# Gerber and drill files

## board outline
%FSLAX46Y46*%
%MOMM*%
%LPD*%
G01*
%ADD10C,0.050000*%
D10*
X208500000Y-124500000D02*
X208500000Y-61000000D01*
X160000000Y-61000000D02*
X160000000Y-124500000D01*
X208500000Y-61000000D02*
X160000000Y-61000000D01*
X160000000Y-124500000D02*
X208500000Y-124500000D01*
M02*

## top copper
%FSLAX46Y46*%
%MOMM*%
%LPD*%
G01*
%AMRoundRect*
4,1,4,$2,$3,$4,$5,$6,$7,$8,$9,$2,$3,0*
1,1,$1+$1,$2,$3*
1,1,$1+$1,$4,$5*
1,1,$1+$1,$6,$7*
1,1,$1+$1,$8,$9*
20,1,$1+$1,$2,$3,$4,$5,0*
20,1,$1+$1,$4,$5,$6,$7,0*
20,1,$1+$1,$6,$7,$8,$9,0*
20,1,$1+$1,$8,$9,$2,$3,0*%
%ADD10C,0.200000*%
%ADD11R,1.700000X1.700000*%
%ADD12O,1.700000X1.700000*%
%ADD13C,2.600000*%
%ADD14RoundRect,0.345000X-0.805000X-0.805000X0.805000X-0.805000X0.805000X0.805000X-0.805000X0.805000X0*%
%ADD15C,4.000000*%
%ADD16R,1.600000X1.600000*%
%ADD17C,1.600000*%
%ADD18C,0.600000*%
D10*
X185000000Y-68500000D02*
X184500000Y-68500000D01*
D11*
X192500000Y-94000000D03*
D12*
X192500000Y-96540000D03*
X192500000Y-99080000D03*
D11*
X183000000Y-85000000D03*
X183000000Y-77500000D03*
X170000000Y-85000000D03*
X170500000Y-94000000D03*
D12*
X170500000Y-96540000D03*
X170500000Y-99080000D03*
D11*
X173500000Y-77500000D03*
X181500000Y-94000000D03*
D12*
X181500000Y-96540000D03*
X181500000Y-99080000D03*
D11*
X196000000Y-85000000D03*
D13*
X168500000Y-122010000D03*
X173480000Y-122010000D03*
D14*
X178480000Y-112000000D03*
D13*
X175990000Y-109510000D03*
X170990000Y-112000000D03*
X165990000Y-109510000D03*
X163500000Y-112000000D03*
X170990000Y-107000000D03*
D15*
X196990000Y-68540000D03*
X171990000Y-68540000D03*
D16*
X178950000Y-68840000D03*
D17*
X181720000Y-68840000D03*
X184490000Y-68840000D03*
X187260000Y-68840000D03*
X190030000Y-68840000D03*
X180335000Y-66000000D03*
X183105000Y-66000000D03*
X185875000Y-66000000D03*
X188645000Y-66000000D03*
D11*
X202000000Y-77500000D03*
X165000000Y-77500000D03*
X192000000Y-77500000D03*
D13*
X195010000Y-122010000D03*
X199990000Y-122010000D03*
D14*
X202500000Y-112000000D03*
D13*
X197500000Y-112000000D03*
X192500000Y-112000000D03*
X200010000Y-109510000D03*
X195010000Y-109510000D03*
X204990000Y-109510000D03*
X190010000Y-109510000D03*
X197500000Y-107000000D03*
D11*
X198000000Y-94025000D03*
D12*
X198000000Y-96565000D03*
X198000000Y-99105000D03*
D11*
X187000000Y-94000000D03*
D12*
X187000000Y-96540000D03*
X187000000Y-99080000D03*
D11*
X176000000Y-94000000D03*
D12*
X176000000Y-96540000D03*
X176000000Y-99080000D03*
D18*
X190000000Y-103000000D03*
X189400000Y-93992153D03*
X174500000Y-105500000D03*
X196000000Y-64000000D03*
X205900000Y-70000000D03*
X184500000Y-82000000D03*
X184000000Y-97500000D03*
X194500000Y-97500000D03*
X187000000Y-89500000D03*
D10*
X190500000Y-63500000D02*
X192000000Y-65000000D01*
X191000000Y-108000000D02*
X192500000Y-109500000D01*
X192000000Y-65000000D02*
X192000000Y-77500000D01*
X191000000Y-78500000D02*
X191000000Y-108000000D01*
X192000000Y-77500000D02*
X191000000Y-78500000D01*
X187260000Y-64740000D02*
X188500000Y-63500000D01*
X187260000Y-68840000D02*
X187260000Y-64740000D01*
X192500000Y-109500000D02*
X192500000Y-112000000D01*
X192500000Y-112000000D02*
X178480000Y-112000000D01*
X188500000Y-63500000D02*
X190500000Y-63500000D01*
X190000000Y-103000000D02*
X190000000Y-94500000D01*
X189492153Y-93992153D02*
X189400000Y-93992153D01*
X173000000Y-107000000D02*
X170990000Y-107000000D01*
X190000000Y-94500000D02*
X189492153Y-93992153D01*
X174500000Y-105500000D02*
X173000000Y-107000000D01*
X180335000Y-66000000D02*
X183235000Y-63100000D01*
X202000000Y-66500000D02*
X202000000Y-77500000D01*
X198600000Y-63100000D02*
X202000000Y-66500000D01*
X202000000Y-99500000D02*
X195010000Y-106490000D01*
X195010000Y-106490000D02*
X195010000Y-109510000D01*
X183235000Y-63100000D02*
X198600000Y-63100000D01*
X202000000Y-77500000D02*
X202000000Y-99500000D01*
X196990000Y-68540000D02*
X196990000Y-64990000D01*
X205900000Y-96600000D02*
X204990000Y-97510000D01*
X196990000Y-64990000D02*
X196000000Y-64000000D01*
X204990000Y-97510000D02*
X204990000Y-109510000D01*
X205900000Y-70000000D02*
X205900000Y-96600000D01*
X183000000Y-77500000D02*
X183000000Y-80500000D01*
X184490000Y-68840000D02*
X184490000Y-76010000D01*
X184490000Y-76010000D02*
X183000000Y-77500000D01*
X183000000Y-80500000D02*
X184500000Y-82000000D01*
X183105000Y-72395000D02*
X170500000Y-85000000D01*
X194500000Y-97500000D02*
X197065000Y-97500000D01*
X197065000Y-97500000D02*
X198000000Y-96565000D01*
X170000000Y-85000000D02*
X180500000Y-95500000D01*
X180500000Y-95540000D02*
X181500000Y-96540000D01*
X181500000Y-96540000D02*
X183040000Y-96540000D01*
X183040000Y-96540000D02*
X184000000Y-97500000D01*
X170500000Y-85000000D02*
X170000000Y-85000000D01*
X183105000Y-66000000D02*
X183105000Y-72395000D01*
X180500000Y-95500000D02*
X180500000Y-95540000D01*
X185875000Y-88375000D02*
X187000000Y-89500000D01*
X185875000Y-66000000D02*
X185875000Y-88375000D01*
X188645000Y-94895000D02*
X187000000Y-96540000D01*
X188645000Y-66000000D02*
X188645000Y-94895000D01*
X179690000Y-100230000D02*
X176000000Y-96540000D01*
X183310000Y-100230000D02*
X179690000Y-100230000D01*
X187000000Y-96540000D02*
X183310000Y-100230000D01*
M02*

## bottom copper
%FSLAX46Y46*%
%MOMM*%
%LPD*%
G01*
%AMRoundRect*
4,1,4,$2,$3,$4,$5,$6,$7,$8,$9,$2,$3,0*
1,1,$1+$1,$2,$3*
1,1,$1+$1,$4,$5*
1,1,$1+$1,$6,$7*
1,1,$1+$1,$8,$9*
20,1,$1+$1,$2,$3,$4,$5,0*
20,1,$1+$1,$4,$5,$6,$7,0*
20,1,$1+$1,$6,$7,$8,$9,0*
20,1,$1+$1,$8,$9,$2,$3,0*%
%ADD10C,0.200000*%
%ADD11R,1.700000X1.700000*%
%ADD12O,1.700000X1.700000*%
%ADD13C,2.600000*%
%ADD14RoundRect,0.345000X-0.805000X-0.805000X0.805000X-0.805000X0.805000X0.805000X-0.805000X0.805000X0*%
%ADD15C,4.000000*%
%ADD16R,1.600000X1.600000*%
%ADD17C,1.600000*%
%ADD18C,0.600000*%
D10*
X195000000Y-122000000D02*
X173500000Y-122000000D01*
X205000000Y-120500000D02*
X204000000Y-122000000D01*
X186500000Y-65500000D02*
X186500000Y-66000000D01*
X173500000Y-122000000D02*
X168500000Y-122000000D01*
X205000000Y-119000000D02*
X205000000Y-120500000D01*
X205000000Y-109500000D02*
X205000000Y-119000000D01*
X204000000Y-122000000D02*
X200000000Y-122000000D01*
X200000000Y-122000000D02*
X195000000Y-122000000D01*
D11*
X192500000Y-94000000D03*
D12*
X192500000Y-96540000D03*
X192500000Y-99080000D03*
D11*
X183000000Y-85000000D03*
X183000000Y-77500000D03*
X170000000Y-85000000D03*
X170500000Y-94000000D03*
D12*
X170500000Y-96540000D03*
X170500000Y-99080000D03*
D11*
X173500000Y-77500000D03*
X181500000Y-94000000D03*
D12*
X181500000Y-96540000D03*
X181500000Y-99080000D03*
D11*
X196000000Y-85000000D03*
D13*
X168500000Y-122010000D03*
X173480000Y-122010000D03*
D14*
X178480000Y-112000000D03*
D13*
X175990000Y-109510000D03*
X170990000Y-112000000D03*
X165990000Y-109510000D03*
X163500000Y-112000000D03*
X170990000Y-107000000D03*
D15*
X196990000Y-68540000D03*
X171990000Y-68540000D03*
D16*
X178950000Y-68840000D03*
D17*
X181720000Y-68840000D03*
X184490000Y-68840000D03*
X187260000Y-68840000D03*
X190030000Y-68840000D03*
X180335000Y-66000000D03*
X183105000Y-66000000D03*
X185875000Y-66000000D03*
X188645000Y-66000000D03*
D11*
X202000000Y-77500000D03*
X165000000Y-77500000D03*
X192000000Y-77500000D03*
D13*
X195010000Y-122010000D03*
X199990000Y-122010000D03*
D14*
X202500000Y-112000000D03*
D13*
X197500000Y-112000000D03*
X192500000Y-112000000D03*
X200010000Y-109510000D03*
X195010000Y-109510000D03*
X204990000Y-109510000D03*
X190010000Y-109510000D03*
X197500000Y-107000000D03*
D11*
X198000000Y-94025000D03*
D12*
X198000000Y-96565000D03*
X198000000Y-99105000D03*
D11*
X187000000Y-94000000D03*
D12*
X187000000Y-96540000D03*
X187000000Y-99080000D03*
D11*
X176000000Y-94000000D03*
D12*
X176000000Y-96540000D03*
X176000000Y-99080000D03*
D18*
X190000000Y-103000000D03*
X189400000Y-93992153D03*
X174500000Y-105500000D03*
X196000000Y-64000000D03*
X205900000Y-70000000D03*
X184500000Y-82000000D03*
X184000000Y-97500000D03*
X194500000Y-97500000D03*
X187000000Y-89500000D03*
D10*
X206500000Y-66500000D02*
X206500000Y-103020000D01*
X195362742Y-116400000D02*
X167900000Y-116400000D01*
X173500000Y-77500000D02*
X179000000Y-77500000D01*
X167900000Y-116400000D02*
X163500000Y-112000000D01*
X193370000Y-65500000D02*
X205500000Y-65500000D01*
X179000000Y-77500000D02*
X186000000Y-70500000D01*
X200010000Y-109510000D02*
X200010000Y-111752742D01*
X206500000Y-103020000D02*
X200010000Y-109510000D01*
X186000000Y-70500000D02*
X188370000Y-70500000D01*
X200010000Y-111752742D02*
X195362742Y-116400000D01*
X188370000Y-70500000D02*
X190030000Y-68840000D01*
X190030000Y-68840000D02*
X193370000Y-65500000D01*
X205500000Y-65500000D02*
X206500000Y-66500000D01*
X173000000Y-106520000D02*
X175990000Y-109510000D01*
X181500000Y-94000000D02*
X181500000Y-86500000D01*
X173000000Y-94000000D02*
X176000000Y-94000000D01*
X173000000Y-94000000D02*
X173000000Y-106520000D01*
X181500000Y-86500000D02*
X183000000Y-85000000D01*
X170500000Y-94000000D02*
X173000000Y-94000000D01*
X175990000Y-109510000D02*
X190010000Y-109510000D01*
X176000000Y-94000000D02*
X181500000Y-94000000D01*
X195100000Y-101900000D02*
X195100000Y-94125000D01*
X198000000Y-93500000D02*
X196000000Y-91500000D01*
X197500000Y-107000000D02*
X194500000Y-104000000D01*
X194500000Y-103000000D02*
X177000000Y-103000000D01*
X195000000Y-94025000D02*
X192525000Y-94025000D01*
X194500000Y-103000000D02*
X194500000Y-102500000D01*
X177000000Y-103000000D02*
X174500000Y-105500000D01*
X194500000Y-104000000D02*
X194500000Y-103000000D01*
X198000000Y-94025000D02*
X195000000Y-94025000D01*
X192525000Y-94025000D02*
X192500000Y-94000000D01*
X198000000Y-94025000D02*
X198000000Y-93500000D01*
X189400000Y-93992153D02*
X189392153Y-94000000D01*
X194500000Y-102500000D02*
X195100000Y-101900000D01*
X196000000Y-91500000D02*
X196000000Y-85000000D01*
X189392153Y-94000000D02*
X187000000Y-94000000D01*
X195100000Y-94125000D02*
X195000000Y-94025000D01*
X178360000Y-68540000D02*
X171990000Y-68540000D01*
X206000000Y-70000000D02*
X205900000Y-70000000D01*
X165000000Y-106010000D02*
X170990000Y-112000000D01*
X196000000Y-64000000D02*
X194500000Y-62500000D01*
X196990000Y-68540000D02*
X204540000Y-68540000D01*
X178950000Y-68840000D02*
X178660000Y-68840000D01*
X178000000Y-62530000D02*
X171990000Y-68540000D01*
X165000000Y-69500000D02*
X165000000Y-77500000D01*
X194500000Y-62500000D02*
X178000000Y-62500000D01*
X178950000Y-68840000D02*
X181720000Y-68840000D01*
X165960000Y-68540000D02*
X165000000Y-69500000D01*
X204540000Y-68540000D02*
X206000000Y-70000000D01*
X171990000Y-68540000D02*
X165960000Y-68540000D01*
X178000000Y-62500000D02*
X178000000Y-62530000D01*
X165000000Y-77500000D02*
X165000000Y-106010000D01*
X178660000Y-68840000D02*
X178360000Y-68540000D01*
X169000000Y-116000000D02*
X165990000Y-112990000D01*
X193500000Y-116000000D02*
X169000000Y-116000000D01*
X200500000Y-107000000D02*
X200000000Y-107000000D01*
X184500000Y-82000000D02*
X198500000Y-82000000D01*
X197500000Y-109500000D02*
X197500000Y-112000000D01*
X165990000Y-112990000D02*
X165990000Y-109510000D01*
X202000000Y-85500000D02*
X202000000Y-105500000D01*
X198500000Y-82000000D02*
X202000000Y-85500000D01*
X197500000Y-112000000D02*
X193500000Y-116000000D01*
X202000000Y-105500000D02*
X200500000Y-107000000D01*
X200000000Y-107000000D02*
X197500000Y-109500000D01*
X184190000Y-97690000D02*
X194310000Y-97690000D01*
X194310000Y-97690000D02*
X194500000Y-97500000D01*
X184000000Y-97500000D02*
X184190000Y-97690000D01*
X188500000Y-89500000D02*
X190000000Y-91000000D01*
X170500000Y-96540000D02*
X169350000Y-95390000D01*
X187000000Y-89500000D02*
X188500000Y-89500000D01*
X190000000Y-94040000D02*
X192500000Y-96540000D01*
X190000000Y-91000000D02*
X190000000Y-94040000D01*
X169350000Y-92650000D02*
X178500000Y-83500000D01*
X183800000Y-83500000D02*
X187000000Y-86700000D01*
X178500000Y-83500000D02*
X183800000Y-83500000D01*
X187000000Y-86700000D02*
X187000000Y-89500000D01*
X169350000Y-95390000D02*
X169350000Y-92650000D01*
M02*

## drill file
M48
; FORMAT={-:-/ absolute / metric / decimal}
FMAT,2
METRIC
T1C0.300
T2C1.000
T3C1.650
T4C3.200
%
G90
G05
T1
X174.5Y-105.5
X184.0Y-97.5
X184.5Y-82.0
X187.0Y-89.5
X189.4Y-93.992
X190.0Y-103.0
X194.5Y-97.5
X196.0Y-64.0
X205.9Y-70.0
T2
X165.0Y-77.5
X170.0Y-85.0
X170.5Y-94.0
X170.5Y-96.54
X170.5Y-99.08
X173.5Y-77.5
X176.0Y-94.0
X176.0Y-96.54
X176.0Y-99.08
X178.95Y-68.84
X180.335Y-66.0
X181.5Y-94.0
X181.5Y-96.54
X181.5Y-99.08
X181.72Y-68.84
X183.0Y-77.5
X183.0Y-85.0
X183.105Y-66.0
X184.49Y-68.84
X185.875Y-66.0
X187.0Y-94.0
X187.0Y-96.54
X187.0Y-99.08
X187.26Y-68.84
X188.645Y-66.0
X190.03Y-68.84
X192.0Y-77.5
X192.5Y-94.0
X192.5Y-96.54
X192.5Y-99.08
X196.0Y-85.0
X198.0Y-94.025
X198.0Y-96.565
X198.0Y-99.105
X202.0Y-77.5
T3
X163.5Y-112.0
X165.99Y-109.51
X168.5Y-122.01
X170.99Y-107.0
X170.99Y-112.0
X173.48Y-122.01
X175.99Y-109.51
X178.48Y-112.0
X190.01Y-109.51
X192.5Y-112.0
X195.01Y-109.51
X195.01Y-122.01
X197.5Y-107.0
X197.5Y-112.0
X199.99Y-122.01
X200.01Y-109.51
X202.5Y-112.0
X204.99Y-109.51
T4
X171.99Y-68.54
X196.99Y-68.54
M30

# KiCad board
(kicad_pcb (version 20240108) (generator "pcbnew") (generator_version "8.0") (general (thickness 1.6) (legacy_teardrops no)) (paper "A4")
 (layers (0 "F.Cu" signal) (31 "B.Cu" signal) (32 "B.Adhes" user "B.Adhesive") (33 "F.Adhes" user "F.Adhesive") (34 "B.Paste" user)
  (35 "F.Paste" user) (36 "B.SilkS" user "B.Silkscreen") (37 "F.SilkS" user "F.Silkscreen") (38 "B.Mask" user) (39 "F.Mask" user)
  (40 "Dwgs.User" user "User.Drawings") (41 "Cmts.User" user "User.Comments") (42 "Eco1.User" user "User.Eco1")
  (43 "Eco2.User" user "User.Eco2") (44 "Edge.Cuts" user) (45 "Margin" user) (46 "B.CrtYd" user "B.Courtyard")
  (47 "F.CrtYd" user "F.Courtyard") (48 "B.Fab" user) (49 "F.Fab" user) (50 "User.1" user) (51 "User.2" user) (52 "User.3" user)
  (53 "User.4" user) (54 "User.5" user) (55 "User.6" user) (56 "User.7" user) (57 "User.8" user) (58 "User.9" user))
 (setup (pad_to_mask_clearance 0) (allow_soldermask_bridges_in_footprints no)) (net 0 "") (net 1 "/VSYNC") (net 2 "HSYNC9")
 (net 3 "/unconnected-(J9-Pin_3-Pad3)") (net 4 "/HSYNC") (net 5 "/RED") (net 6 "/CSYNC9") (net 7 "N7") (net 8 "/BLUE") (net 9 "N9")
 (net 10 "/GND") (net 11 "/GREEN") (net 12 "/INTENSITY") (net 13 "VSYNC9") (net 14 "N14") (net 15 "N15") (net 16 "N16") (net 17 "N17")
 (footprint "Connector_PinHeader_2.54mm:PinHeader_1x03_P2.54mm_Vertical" (layer "F.Cu") (at 192.5 94)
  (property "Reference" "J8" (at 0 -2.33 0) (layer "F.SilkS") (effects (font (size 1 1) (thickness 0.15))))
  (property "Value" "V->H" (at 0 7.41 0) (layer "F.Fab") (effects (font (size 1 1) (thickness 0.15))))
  (pad "1" thru_hole rect (at 0 0) (size 1.7 1.7) (drill 1) (layers "*.Cu" "*.Mask") (remove_unused_layers no) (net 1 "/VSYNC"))
  (pad "2" thru_hole oval (at 0 2.54) (size 1.7 1.7) (drill 1) (layers "*.Cu" "*.Mask") (remove_unused_layers no) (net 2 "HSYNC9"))
  (pad "3" thru_hole oval (at 0 5.08) (size 1.7 1.7) (drill 1) (layers "*.Cu" "*.Mask") (remove_unused_layers no)
   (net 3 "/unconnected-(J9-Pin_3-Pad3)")))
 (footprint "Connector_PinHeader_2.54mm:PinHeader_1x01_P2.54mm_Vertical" (layer "F.Cu") (at 183 85)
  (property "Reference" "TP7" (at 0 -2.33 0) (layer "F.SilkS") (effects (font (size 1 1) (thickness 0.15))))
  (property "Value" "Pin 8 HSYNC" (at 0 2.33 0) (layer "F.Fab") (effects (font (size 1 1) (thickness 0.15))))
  (pad "1" thru_hole rect (at 0 0) (size 1.7 1.7) (drill 1) (layers "*.Cu" "*.Mask") (remove_unused_layers no) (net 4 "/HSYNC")))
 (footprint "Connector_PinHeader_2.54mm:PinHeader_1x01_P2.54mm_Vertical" (layer "F.Cu") (at 183 77.5)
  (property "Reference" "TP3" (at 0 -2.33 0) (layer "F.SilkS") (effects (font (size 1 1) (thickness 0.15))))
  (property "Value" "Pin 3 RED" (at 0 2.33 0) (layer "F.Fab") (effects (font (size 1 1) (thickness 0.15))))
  (pad "1" thru_hole rect (at 0 0) (size 1.7 1.7) (drill 1) (layers "*.Cu" "*.Mask") (remove_unused_layers no) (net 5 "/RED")))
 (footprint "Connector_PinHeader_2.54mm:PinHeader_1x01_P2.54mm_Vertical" (layer "F.Cu") (at 170 85)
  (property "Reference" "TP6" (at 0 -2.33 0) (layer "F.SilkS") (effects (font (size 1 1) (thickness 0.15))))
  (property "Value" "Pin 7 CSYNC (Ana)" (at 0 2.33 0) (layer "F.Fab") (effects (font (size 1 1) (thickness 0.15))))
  (pad "1" thru_hole rect (at 0 0) (size 1.7 1.7) (drill 1) (layers "*.Cu" "*.Mask") (remove_unused_layers no) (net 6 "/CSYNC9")))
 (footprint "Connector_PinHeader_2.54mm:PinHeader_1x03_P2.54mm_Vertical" (layer "F.Cu") (at 170.5 94)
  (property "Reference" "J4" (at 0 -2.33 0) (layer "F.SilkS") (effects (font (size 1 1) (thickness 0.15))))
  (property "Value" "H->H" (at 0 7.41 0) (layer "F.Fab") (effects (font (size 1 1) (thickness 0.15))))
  (pad "1" thru_hole rect (at 0 0) (size 1.7 1.7) (drill 1) (layers "*.Cu" "*.Mask") (remove_unused_layers no) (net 4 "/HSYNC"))
  (pad "2" thru_hole oval (at 0 2.54) (size 1.7 1.7) (drill 1) (layers "*.Cu" "*.Mask") (remove_unused_layers no) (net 2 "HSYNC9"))
  (pad "3" thru_hole oval (at 0 5.08) (size 1.7 1.7) (drill 1) (layers "*.Cu" "*.Mask") (remove_unused_layers no) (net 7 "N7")))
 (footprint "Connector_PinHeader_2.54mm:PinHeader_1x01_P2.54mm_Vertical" (layer "F.Cu") (at 173.5 77.5)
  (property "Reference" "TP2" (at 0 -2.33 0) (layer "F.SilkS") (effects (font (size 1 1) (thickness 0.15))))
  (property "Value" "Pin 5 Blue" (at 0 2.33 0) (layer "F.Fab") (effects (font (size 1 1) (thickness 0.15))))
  (pad "1" thru_hole rect (at 0 0) (size 1.7 1.7) (drill 1) (layers "*.Cu" "*.Mask") (remove_unused_layers no) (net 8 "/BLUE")))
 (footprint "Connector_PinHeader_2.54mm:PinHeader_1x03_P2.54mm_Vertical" (layer "F.Cu") (at 181.5 94)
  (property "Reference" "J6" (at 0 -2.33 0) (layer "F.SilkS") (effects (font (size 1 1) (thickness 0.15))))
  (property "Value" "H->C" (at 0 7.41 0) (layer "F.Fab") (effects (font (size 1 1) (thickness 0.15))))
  (pad "1" thru_hole rect (at 0 0) (size 1.7 1.7) (drill 1) (layers "*.Cu" "*.Mask") (remove_unused_layers no) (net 4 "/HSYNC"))
  (pad "2" thru_hole oval (at 0 2.54) (size 1.7 1.7) (drill 1) (layers "*.Cu" "*.Mask") (remove_unused_layers no) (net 6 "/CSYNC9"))
  (pad "3" thru_hole oval (at 0 5.08) (size 1.7 1.7) (drill 1) (layers "*.Cu" "*.Mask") (remove_unused_layers no) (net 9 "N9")))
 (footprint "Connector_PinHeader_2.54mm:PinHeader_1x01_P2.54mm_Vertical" (layer "F.Cu") (at 196 85)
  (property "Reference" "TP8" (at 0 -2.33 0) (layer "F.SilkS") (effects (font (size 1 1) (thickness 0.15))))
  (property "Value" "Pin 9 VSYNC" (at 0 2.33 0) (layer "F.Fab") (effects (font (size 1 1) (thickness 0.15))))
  (pad "1" thru_hole rect (at 0 0) (size 1.7 1.7) (drill 1) (layers "*.Cu" "*.Mask") (remove_unused_layers no) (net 1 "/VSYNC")))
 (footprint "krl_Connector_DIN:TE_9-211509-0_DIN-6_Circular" (layer "F.Cu") (at 178.48 112)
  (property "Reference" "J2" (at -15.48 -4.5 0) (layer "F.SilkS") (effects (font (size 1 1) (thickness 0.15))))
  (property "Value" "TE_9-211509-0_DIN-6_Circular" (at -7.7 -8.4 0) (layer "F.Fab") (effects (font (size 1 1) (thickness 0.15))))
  (pad "0" thru_hole circle (at -9.98 10.01) (size 2.6 2.6) (drill 1.65) (layers "*.Cu" "*.Mask") (remove_unused_layers no) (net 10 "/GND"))
  (pad "0" thru_hole circle (at -5 10.01) (size 2.6 2.6) (drill 1.65) (layers "*.Cu" "*.Mask") (remove_unused_layers no) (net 10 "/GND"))
  (pad "1" thru_hole roundrect (at 0 0) (size 2.3 2.3) (drill 1.65) (layers "*.Cu" "*.Mask") (remove_unused_layers no)
   (roundrect_rratio 0.15) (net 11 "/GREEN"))
  (pad "2" thru_hole circle (at -2.49 -2.49) (size 2.6 2.6) (drill 1.65) (layers "*.Cu" "*.Mask") (remove_unused_layers no) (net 4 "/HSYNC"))
  (pad "3" thru_hole circle (at -7.49 0) (size 2.6 2.6) (drill 1.65) (layers "*.Cu" "*.Mask") (remove_unused_layers no) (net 10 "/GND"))
  (pad "4" thru_hole circle (at -12.49 -2.49) (size 2.6 2.6) (drill 1.65) (layers "*.Cu" "*.Mask") (remove_unused_layers no) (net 5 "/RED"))
  (pad "5" thru_hole circle (at -14.98 0) (size 2.6 2.6) (drill 1.65) (layers "*.Cu" "*.Mask") (remove_unused_layers no) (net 8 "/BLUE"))
  (pad "6" thru_hole circle (at -7.49 -5) (size 2.6 2.6) (drill 1.65) (layers "*.Cu" "*.Mask") (remove_unused_layers no) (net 1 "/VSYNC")))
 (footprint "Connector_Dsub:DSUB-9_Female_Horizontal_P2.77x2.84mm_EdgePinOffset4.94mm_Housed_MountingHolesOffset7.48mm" (layer "F.Cu")
  (at 178.95 68.84 180)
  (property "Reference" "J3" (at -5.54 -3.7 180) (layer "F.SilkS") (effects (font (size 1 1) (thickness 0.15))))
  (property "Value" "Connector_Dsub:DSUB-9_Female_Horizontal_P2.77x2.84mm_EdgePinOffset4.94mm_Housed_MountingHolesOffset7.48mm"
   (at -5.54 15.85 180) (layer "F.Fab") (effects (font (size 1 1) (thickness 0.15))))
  (pad "0" thru_hole circle (at -18.04 0.3 180) (size 4 4) (drill 3.2) (layers "*.Cu" "*.Mask") (remove_unused_layers no) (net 10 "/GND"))
  (pad "0" thru_hole circle (at 6.96 0.3 180) (size 4 4) (drill 3.2) (layers "*.Cu" "*.Mask") (remove_unused_layers no) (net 10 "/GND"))
  (pad "1" thru_hole rect (at 0 0 180) (size 1.6 1.6) (drill 1) (layers "*.Cu" "*.Mask") (remove_unused_layers no) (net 10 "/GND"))
  (pad "2" thru_hole circle (at -2.77 0 180) (size 1.6 1.6) (drill 1) (layers "*.Cu" "*.Mask") (remove_unused_layers no) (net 10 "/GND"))
  (pad "3" thru_hole circle (at -5.54 0 180) (size 1.6 1.6) (drill 1) (layers "*.Cu" "*.Mask") (remove_unused_layers no) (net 5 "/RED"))
  (pad "4" thru_hole circle (at -8.31 0 180) (size 1.6 1.6) (drill 1) (layers "*.Cu" "*.Mask") (remove_unused_layers no) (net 11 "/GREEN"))
  (pad "5" thru_hole circle (at -11.08 0 180) (size 1.6 1.6) (drill 1) (layers "*.Cu" "*.Mask") (remove_unused_layers no) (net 8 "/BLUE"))
  (pad "6" thru_hole circle (at -1.385 2.84 180) (size 1.6 1.6) (drill 1) (layers "*.Cu" "*.Mask") (remove_unused_layers no)
   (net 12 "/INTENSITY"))
  (pad "7" thru_hole circle (at -4.155 2.84 180) (size 1.6 1.6) (drill 1) (layers "*.Cu" "*.Mask") (remove_unused_layers no)
   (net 6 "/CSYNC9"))
  (pad "8" thru_hole circle (at -6.925 2.84 180) (size 1.6 1.6) (drill 1) (layers "*.Cu" "*.Mask") (remove_unused_layers no)
   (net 2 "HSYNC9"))
  (pad "9" thru_hole circle (at -9.695 2.84 180) (size 1.6 1.6) (drill 1) (layers "*.Cu" "*.Mask") (remove_unused_layers no)
   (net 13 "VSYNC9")))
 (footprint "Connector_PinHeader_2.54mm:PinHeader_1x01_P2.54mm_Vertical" (layer "F.Cu") (at 202 77.5)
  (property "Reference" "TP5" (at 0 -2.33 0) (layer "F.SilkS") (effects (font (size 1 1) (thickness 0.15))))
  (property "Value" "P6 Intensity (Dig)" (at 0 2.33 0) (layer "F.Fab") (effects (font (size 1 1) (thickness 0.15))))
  (pad "1" thru_hole rect (at 0 0) (size 1.7 1.7) (drill 1) (layers "*.Cu" "*.Mask") (remove_unused_layers no) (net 12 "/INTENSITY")))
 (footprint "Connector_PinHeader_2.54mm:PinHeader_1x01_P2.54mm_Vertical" (layer "F.Cu") (at 165 77.5)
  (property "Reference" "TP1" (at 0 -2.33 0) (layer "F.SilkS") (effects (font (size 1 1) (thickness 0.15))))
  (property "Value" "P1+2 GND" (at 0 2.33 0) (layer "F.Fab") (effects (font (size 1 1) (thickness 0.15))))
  (pad "1" thru_hole rect (at 0 0) (size 1.7 1.7) (drill 1) (layers "*.Cu" "*.Mask") (remove_unused_layers no) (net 10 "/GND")))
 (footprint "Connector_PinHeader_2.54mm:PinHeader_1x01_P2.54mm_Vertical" (layer "F.Cu") (at 192 77.5)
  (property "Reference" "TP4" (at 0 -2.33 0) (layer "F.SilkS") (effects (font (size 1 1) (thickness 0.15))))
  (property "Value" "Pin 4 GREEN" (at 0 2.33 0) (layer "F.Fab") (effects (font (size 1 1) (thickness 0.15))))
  (pad "1" thru_hole rect (at 0 0) (size 1.7 1.7) (drill 1) (layers "*.Cu" "*.Mask") (remove_unused_layers no) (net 11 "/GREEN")))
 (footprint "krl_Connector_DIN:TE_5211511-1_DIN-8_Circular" (layer "F.Cu") (at 202.5 112)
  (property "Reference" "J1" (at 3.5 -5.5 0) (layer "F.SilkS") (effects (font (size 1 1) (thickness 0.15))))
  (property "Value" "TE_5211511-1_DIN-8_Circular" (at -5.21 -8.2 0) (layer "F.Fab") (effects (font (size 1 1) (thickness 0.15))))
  (pad "0" thru_hole circle (at -7.49 10.01) (size 2.6 2.6) (drill 1.65) (layers "*.Cu" "*.Mask") (remove_unused_layers no) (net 10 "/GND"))
  (pad "0" thru_hole circle (at -2.51 10.01) (size 2.6 2.6) (drill 1.65) (layers "*.Cu" "*.Mask") (remove_unused_layers no) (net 10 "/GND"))
  (pad "1" thru_hole roundrect (at 0 0) (size 2.3 2.3) (drill 1.65) (layers "*.Cu" "*.Mask") (remove_unused_layers no)
   (roundrect_rratio 0.15) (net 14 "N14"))
  (pad "2" thru_hole circle (at -5 0) (size 2.6 2.6) (drill 1.65) (layers "*.Cu" "*.Mask") (remove_unused_layers no) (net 5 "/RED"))
  (pad "3" thru_hole circle (at -10 0) (size 2.6 2.6) (drill 1.65) (layers "*.Cu" "*.Mask") (remove_unused_layers no) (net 11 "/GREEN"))
  (pad "4" thru_hole circle (at -2.49 -2.49) (size 2.6 2.6) (drill 1.65) (layers "*.Cu" "*.Mask") (remove_unused_layers no) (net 8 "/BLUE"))
  (pad "5" thru_hole circle (at -7.49 -2.49) (size 2.6 2.6) (drill 1.65) (layers "*.Cu" "*.Mask") (remove_unused_layers no)
   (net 12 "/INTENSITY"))
  (pad "6" thru_hole circle (at 2.49 -2.49) (size 2.6 2.6) (drill 1.65) (layers "*.Cu" "*.Mask") (remove_unused_layers no) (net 10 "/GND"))
  (pad "7" thru_hole circle (at -12.49 -2.49) (size 2.6 2.6) (drill 1.65) (layers "*.Cu" "*.Mask") (remove_unused_layers no)
   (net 4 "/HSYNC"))
  (pad "8" thru_hole circle (at -5 -5) (size 2.6 2.6) (drill 1.65) (layers "*.Cu" "*.Mask") (remove_unused_layers no) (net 1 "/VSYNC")))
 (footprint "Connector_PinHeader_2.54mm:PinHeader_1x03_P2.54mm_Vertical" (layer "F.Cu") (at 198 94.025)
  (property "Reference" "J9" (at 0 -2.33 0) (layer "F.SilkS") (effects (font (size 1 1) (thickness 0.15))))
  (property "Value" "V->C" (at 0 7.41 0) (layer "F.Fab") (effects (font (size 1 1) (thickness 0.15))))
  (pad "1" thru_hole rect (at 0 0) (size 1.7 1.7) (drill 1) (layers "*.Cu" "*.Mask") (remove_unused_layers no) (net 1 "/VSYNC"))
  (pad "2" thru_hole oval (at 0 2.54) (size 1.7 1.7) (drill 1) (layers "*.Cu" "*.Mask") (remove_unused_layers no) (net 6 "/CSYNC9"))
  (pad "3" thru_hole oval (at 0 5.08) (size 1.7 1.7) (drill 1) (layers "*.Cu" "*.Mask") (remove_unused_layers no) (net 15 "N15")))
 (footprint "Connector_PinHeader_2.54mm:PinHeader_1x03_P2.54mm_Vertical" (layer "F.Cu") (at 187 94)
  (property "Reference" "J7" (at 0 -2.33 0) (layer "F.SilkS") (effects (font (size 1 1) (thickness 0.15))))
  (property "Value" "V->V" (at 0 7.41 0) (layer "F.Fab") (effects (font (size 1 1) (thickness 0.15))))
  (pad "1" thru_hole rect (at 0 0) (size 1.7 1.7) (drill 1) (layers "*.Cu" "*.Mask") (remove_unused_layers no) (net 1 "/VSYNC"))
  (pad "2" thru_hole oval (at 0 2.54) (size 1.7 1.7) (drill 1) (layers "*.Cu" "*.Mask") (remove_unused_layers no) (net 13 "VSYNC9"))
  (pad "3" thru_hole oval (at 0 5.08) (size 1.7 1.7) (drill 1) (layers "*.Cu" "*.Mask") (remove_unused_layers no) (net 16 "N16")))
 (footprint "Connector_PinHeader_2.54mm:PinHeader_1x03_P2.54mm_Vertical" (layer "F.Cu") (at 176 94)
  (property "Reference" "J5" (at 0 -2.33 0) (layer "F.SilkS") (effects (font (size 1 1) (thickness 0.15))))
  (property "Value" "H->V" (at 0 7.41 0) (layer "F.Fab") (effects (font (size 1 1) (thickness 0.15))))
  (pad "1" thru_hole rect (at 0 0) (size 1.7 1.7) (drill 1) (layers "*.Cu" "*.Mask") (remove_unused_layers no) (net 4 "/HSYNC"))
  (pad "2" thru_hole oval (at 0 2.54) (size 1.7 1.7) (drill 1) (layers "*.Cu" "*.Mask") (remove_unused_layers no) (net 13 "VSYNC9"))
  (pad "3" thru_hole oval (at 0 5.08) (size 1.7 1.7) (drill 1) (layers "*.Cu" "*.Mask") (remove_unused_layers no) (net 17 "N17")))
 (gr_line (start 185 68.5) (end 184.5 68.5) (stroke (width 0.2) (type default)) (layer "F.Cu") (net 5))
 (gr_line (start 195 122) (end 173.5 122) (stroke (width 0.2) (type default)) (layer "B.Cu") (net 10))
 (gr_line (start 205 120.5) (end 204 122) (stroke (width 0.2) (type default)) (layer "B.Cu") (net 10))
 (gr_line (start 186.5 65.5) (end 186.5 66) (stroke (width 0.2) (type default)) (layer "B.Cu") (net 2))
 (gr_line (start 173.5 122) (end 168.5 122) (stroke (width 0.2) (type default)) (layer "B.Cu") (net 10))
 (gr_line (start 205 119) (end 205 120.5) (stroke (width 0.2) (type default)) (layer "B.Cu") (net 10))
 (gr_line (start 205 109.5) (end 205 119) (stroke (width 0.2) (type default)) (layer "B.Cu") (net 10))
 (gr_line (start 204 122) (end 200 122) (stroke (width 0.2) (type default)) (layer "B.Cu") (net 10))
 (gr_line (start 200 122) (end 195 122) (stroke (width 0.2) (type default)) (layer "B.Cu") (net 10))
 (gr_line (start 208.5 124.5) (end 208.5 61) (stroke (width 0.05) (type default)) (layer "Edge.Cuts"))
 (gr_line (start 160 61) (end 160 124.5) (stroke (width 0.05) (type default)) (layer "Edge.Cuts"))
 (gr_line (start 208.5 61) (end 160 61) (stroke (width 0.05) (type default)) (layer "Edge.Cuts"))
 (gr_line (start 160 124.5) (end 208.5 124.5) (stroke (width 0.05) (type default)) (layer "Edge.Cuts"))
 (segment (start 206.5 66.5) (end 206.5 103.02) (width 0.2) (layer "B.Cu") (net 8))
 (segment (start 195.362742 116.4) (end 167.9 116.4) (width 0.2) (layer "B.Cu") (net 8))
 (segment (start 173.5 77.5) (end 179 77.5) (width 0.2) (layer "B.Cu") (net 8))
 (segment (start 167.9 116.4) (end 163.5 112) (width 0.2) (layer "B.Cu") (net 8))
 (segment (start 193.37 65.5) (end 205.5 65.5) (width 0.2) (layer "B.Cu") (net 8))
 (segment (start 179 77.5) (end 186 70.5) (width 0.2) (layer "B.Cu") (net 8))
 (segment (start 200.01 109.51) (end 200.01 111.752742) (width 0.2) (layer "B.Cu") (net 8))
 (segment (start 206.5 103.02) (end 200.01 109.51) (width 0.2) (layer "B.Cu") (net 8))
 (segment (start 186 70.5) (end 188.37 70.5) (width 0.2) (layer "B.Cu") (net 8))
 (segment (start 200.01 111.752742) (end 195.362742 116.4) (width 0.2) (layer "B.Cu") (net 8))
 (segment (start 188.37 70.5) (end 190.03 68.84) (width 0.2) (layer "B.Cu") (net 8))
 (segment (start 190.03 68.84) (end 193.37 65.5) (width 0.2) (layer "B.Cu") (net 8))
 (segment (start 205.5 65.5) (end 206.5 66.5) (width 0.2) (layer "B.Cu") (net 8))
 (segment (start 173 106.52) (end 175.99 109.51) (width 0.2) (layer "B.Cu") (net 4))
 (segment (start 181.5 94) (end 181.5 86.5) (width 0.2) (layer "B.Cu") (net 4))
 (segment (start 173 94) (end 176 94) (width 0.2) (layer "B.Cu") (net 4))
 (segment (start 173 94) (end 173 106.52) (width 0.2) (layer "B.Cu") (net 4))
 (segment (start 181.5 86.5) (end 183 85) (width 0.2) (layer "B.Cu") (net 4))
 (segment (start 170.5 94) (end 173 94) (width 0.2) (layer "B.Cu") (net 4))
 (segment (start 175.99 109.51) (end 190.01 109.51) (width 0.2) (layer "B.Cu") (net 4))
 (segment (start 176 94) (end 181.5 94) (width 0.2) (layer "B.Cu") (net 4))
 (segment (start 190.5 63.5) (end 192 65) (width 0.2) (layer "F.Cu") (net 11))
 (segment (start 191 108) (end 192.5 109.5) (width 0.2) (layer "F.Cu") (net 11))
 (segment (start 192 65) (end 192 77.5) (width 0.2) (layer "F.Cu") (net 11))
 (segment (start 191 78.5) (end 191 108) (width 0.2) (layer "F.Cu") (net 11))
 (segment (start 192 77.5) (end 191 78.5) (width 0.2) (layer "F.Cu") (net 11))
 (segment (start 187.26 64.74) (end 188.5 63.5) (width 0.2) (layer "F.Cu") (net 11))
 (segment (start 187.26 68.84) (end 187.26 64.74) (width 0.2) (layer "F.Cu") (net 11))
 (segment (start 192.5 109.5) (end 192.5 112) (width 0.2) (layer "F.Cu") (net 11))
 (segment (start 192.5 112) (end 178.48 112) (width 0.2) (layer "F.Cu") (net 11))
 (segment (start 188.5 63.5) (end 190.5 63.5) (width 0.2) (layer "F.Cu") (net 11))
 (segment (start 190 103) (end 190 94.5) (width 0.2) (layer "F.Cu") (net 1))
 (segment (start 189.492153 93.992153) (end 189.4 93.992153) (width 0.2) (layer "F.Cu") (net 1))
 (segment (start 173 107) (end 170.99 107) (width 0.2) (layer "F.Cu") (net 1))
 (segment (start 190 94.5) (end 189.492153 93.992153) (width 0.2) (layer "F.Cu") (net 1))
 (segment (start 174.5 105.5) (end 173 107) (width 0.2) (layer "F.Cu") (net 1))
 (via (at 190 103) (size 0.6) (drill 0.3) (layers "F.Cu" "B.Cu") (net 1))
 (via (at 189.4 93.992153) (size 0.6) (drill 0.3) (layers "F.Cu" "B.Cu") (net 1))
 (via (at 174.5 105.5) (size 0.6) (drill 0.3) (layers "F.Cu" "B.Cu") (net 1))
 (segment (start 195.1 101.9) (end 195.1 94.125) (width 0.2) (layer "B.Cu") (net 1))
 (segment (start 198 93.5) (end 196 91.5) (width 0.2) (layer "B.Cu") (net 1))
 (segment (start 197.5 107) (end 194.5 104) (width 0.2) (layer "B.Cu") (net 1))
 (segment (start 194.5 103) (end 177 103) (width 0.2) (layer "B.Cu") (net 1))
 (segment (start 195 94.025) (end 192.525 94.025) (width 0.2) (layer "B.Cu") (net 1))
 (segment (start 194.5 103) (end 194.5 102.5) (width 0.2) (layer "B.Cu") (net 1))
 (segment (start 177 103) (end 174.5 105.5) (width 0.2) (layer "B.Cu") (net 1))
 (segment (start 194.5 104) (end 194.5 103) (width 0.2) (layer "B.Cu") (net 1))
 (segment (start 198 94.025) (end 195 94.025) (width 0.2) (layer "B.Cu") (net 1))
 (segment (start 192.525 94.025) (end 192.5 94) (width 0.2) (layer "B.Cu") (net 1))
 (segment (start 198 94.025) (end 198 93.5) (width 0.2) (layer "B.Cu") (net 1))
 (segment (start 189.4 93.992153) (end 189.392153 94) (width 0.2) (layer "B.Cu") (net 1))
 (segment (start 194.5 102.5) (end 195.1 101.9) (width 0.2) (layer "B.Cu") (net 1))
 (segment (start 196 91.5) (end 196 85) (width 0.2) (layer "B.Cu") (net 1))
 (segment (start 189.392153 94) (end 187 94) (width 0.2) (layer "B.Cu") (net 1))
 (segment (start 195.1 94.125) (end 195 94.025) (width 0.2) (layer "B.Cu") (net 1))
 (segment (start 180.335 66) (end 183.235 63.1) (width 0.2) (layer "F.Cu") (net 12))
 (segment (start 202 66.5) (end 202 77.5) (width 0.2) (layer "F.Cu") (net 12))
 (segment (start 198.6 63.1) (end 202 66.5) (width 0.2) (layer "F.Cu") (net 12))
 (segment (start 202 99.5) (end 195.01 106.49) (width 0.2) (layer "F.Cu") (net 12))
 (segment (start 195.01 106.49) (end 195.01 109.51) (width 0.2) (layer "F.Cu") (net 12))
 (segment (start 183.235 63.1) (end 198.6 63.1) (width 0.2) (layer "F.Cu") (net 12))
 (segment (start 202 77.5) (end 202 99.5) (width 0.2) (layer "F.Cu") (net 12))
 (segment (start 196.99 68.54) (end 196.99 64.99) (width 0.2) (layer "F.Cu") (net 10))
 (segment (start 205.9 96.6) (end 204.99 97.51) (width 0.2) (layer "F.Cu") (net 10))
 (segment (start 196.99 64.99) (end 196 64) (width 0.2) (layer "F.Cu") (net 10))
 (segment (start 204.99 97.51) (end 204.99 109.51) (width 0.2) (layer "F.Cu") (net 10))
 (segment (start 205.9 70) (end 205.9 96.6) (width 0.2) (layer "F.Cu") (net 10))
 (via (at 196 64) (size 0.6) (drill 0.3) (layers "F.Cu" "B.Cu") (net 10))
 (via (at 205.9 70) (size 0.6) (drill 0.3) (layers "F.Cu" "B.Cu") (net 10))
 (segment (start 178.36 68.54) (end 171.99 68.54) (width 0.2) (layer "B.Cu") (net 10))
 (segment (start 206 70) (end 205.9 70) (width 0.2) (layer "B.Cu") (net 10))
 (segment (start 165 106.01) (end 170.99 112) (width 0.2) (layer "B.Cu") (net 10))
 (segment (start 196 64) (end 194.5 62.5) (width 0.2) (layer "B.Cu") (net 10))
 (segment (start 196.99 68.54) (end 204.54 68.54) (width 0.2) (layer "B.Cu") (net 10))
 (segment (start 178.95 68.84) (end 178.66 68.84) (width 0.2) (layer "B.Cu") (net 10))
 (segment (start 178 62.53) (end 171.99 68.54) (width 0.2) (layer "B.Cu") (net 10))
 (segment (start 165 69.5) (end 165 77.5) (width 0.2) (layer "B.Cu") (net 10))
 (segment (start 194.5 62.5) (end 178 62.5) (width 0.2) (layer "B.Cu") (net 10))
 (segment (start 178.95 68.84) (end 181.72 68.84) (width 0.2) (layer "B.Cu") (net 10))
 (segment (start 165.96 68.54) (end 165 69.5) (width 0.2) (layer "B.Cu") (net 10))
 (segment (start 204.54 68.54) (end 206 70) (width 0.2) (layer "B.Cu") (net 10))
 (segment (start 171.99 68.54) (end 165.96 68.54) (width 0.2) (layer "B.Cu") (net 10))
 (segment (start 178 62.5) (end 178 62.53) (width 0.2) (layer "B.Cu") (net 10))
 (segment (start 165 77.5) (end 165 106.01) (width 0.2) (layer "B.Cu") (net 10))
 (segment (start 178.66 68.84) (end 178.36 68.54) (width 0.2) (layer "B.Cu") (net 10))
 (segment (start 183 77.5) (end 183 80.5) (width 0.2) (layer "F.Cu") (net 5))
 (segment (start 184.49 68.84) (end 184.49 76.01) (width 0.2) (layer "F.Cu") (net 5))
 (segment (start 184.49 76.01) (end 183 77.5) (width 0.2) (layer "F.Cu") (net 5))
 (segment (start 183 80.5) (end 184.5 82) (width 0.2) (layer "F.Cu") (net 5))
 (via (at 184.5 82) (size 0.6) (drill 0.3) (layers "F.Cu" "B.Cu") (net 5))
 (segment (start 169 116) (end 165.99 112.99) (width 0.2) (layer "B.Cu") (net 5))
 (segment (start 193.5 116) (end 169 116) (width 0.2) (layer "B.Cu") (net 5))
 (segment (start 200.5 107) (end 200 107) (width 0.2) (layer "B.Cu") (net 5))
 (segment (start 184.5 82) (end 198.5 82) (width 0.2) (layer "B.Cu") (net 5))
 (segment (start 197.5 109.5) (end 197.5 112) (width 0.2) (layer "B.Cu") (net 5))
 (segment (start 165.99 112.99) (end 165.99 109.51) (width 0.2) (layer "B.Cu") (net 5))
 (segment (start 202 85.5) (end 202 105.5) (width 0.2) (layer "B.Cu") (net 5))
 (segment (start 198.5 82) (end 202 85.5) (width 0.2) (layer "B.Cu") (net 5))
 (segment (start 197.5 112) (end 193.5 116) (width 0.2) (layer "B.Cu") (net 5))
 (segment (start 202 105.5) (end 200.5 107) (width 0.2) (layer "B.Cu") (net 5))
 (segment (start 200 107) (end 197.5 109.5) (width 0.2) (layer "B.Cu") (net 5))
 (segment (start 183.105 72.395) (end 170.5 85) (width 0.2) (layer "F.Cu") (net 6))
 (segment (start 194.5 97.5) (end 197.065 97.5) (width 0.2) (layer "F.Cu") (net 6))
 (segment (start 197.065 97.5) (end 198 96.565) (width 0.2) (layer "F.Cu") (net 6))
 (segment (start 170 85) (end 180.5 95.5) (width 0.2) (layer "F.Cu") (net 6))
 (segment (start 180.5 95.54) (end 181.5 96.54) (width 0.2) (layer "F.Cu") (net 6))
 (segment (start 181.5 96.54) (end 183.04 96.54) (width 0.2) (layer "F.Cu") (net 6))
 (segment (start 183.04 96.54) (end 184 97.5) (width 0.2) (layer "F.Cu") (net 6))
 (segment (start 170.5 85) (end 170 85) (width 0.2) (layer "F.Cu") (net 6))
 (segment (start 183.105 66) (end 183.105 72.395) (width 0.2) (layer "F.Cu") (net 6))
 (segment (start 180.5 95.5) (end 180.5 95.54) (width 0.2) (layer "F.Cu") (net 6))
 (via (at 184 97.5) (size 0.6) (drill 0.3) (layers "F.Cu" "B.Cu") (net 6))
 (via (at 194.5 97.5) (size 0.6) (drill 0.3) (layers "F.Cu" "B.Cu") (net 6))
 (segment (start 184.19 97.69) (end 194.31 97.69) (width 0.2) (layer "B.Cu") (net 6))
 (segment (start 194.31 97.69) (end 194.5 97.5) (width 0.2) (layer "B.Cu") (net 6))
 (segment (start 184 97.5) (end 184.19 97.69) (width 0.2) (layer "B.Cu") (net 6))
 (segment (start 185.875 88.375) (end 187 89.5) (width 0.2) (layer "F.Cu") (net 2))
 (segment (start 185.875 66) (end 185.875 88.375) (width 0.2) (layer "F.Cu") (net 2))
 (via (at 187 89.5) (size 0.6) (drill 0.3) (layers "F.Cu" "B.Cu") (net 2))
 (segment (start 188.5 89.5) (end 190 91) (width 0.2) (layer "B.Cu") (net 2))
 (segment (start 170.5 96.54) (end 169.35 95.39) (width 0.2) (layer "B.Cu") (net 2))
 (segment (start 187 89.5) (end 188.5 89.5) (width 0.2) (layer "B.Cu") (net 2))
 (segment (start 190 94.04) (end 192.5 96.54) (width 0.2) (layer "B.Cu") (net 2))
 (segment (start 190 91) (end 190 94.04) (width 0.2) (layer "B.Cu") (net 2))
 (segment (start 169.35 92.65) (end 178.5 83.5) (width 0.2) (layer "B.Cu") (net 2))
 (segment (start 183.8 83.5) (end 187 86.7) (width 0.2) (layer "B.Cu") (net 2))
 (segment (start 178.5 83.5) (end 183.8 83.5) (width 0.2) (layer "B.Cu") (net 2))
 (segment (start 187 86.7) (end 187 89.5) (width 0.2) (layer "B.Cu") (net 2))
 (segment (start 169.35 95.39) (end 169.35 92.65) (width 0.2) (layer "B.Cu") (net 2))
 (segment (start 188.645 94.895) (end 187 96.54) (width 0.2) (layer "F.Cu") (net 13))
 (segment (start 188.645 66) (end 188.645 94.895) (width 0.2) (layer "F.Cu") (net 13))
 (segment (start 179.69 100.23) (end 176 96.54) (width 0.2) (layer "F.Cu") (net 13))
 (segment (start 183.31 100.23) (end 179.69 100.23) (width 0.2) (layer "F.Cu") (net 13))
 (segment (start 187 96.54) (end 183.31 100.23) (width 0.2) (layer "F.Cu") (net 13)))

